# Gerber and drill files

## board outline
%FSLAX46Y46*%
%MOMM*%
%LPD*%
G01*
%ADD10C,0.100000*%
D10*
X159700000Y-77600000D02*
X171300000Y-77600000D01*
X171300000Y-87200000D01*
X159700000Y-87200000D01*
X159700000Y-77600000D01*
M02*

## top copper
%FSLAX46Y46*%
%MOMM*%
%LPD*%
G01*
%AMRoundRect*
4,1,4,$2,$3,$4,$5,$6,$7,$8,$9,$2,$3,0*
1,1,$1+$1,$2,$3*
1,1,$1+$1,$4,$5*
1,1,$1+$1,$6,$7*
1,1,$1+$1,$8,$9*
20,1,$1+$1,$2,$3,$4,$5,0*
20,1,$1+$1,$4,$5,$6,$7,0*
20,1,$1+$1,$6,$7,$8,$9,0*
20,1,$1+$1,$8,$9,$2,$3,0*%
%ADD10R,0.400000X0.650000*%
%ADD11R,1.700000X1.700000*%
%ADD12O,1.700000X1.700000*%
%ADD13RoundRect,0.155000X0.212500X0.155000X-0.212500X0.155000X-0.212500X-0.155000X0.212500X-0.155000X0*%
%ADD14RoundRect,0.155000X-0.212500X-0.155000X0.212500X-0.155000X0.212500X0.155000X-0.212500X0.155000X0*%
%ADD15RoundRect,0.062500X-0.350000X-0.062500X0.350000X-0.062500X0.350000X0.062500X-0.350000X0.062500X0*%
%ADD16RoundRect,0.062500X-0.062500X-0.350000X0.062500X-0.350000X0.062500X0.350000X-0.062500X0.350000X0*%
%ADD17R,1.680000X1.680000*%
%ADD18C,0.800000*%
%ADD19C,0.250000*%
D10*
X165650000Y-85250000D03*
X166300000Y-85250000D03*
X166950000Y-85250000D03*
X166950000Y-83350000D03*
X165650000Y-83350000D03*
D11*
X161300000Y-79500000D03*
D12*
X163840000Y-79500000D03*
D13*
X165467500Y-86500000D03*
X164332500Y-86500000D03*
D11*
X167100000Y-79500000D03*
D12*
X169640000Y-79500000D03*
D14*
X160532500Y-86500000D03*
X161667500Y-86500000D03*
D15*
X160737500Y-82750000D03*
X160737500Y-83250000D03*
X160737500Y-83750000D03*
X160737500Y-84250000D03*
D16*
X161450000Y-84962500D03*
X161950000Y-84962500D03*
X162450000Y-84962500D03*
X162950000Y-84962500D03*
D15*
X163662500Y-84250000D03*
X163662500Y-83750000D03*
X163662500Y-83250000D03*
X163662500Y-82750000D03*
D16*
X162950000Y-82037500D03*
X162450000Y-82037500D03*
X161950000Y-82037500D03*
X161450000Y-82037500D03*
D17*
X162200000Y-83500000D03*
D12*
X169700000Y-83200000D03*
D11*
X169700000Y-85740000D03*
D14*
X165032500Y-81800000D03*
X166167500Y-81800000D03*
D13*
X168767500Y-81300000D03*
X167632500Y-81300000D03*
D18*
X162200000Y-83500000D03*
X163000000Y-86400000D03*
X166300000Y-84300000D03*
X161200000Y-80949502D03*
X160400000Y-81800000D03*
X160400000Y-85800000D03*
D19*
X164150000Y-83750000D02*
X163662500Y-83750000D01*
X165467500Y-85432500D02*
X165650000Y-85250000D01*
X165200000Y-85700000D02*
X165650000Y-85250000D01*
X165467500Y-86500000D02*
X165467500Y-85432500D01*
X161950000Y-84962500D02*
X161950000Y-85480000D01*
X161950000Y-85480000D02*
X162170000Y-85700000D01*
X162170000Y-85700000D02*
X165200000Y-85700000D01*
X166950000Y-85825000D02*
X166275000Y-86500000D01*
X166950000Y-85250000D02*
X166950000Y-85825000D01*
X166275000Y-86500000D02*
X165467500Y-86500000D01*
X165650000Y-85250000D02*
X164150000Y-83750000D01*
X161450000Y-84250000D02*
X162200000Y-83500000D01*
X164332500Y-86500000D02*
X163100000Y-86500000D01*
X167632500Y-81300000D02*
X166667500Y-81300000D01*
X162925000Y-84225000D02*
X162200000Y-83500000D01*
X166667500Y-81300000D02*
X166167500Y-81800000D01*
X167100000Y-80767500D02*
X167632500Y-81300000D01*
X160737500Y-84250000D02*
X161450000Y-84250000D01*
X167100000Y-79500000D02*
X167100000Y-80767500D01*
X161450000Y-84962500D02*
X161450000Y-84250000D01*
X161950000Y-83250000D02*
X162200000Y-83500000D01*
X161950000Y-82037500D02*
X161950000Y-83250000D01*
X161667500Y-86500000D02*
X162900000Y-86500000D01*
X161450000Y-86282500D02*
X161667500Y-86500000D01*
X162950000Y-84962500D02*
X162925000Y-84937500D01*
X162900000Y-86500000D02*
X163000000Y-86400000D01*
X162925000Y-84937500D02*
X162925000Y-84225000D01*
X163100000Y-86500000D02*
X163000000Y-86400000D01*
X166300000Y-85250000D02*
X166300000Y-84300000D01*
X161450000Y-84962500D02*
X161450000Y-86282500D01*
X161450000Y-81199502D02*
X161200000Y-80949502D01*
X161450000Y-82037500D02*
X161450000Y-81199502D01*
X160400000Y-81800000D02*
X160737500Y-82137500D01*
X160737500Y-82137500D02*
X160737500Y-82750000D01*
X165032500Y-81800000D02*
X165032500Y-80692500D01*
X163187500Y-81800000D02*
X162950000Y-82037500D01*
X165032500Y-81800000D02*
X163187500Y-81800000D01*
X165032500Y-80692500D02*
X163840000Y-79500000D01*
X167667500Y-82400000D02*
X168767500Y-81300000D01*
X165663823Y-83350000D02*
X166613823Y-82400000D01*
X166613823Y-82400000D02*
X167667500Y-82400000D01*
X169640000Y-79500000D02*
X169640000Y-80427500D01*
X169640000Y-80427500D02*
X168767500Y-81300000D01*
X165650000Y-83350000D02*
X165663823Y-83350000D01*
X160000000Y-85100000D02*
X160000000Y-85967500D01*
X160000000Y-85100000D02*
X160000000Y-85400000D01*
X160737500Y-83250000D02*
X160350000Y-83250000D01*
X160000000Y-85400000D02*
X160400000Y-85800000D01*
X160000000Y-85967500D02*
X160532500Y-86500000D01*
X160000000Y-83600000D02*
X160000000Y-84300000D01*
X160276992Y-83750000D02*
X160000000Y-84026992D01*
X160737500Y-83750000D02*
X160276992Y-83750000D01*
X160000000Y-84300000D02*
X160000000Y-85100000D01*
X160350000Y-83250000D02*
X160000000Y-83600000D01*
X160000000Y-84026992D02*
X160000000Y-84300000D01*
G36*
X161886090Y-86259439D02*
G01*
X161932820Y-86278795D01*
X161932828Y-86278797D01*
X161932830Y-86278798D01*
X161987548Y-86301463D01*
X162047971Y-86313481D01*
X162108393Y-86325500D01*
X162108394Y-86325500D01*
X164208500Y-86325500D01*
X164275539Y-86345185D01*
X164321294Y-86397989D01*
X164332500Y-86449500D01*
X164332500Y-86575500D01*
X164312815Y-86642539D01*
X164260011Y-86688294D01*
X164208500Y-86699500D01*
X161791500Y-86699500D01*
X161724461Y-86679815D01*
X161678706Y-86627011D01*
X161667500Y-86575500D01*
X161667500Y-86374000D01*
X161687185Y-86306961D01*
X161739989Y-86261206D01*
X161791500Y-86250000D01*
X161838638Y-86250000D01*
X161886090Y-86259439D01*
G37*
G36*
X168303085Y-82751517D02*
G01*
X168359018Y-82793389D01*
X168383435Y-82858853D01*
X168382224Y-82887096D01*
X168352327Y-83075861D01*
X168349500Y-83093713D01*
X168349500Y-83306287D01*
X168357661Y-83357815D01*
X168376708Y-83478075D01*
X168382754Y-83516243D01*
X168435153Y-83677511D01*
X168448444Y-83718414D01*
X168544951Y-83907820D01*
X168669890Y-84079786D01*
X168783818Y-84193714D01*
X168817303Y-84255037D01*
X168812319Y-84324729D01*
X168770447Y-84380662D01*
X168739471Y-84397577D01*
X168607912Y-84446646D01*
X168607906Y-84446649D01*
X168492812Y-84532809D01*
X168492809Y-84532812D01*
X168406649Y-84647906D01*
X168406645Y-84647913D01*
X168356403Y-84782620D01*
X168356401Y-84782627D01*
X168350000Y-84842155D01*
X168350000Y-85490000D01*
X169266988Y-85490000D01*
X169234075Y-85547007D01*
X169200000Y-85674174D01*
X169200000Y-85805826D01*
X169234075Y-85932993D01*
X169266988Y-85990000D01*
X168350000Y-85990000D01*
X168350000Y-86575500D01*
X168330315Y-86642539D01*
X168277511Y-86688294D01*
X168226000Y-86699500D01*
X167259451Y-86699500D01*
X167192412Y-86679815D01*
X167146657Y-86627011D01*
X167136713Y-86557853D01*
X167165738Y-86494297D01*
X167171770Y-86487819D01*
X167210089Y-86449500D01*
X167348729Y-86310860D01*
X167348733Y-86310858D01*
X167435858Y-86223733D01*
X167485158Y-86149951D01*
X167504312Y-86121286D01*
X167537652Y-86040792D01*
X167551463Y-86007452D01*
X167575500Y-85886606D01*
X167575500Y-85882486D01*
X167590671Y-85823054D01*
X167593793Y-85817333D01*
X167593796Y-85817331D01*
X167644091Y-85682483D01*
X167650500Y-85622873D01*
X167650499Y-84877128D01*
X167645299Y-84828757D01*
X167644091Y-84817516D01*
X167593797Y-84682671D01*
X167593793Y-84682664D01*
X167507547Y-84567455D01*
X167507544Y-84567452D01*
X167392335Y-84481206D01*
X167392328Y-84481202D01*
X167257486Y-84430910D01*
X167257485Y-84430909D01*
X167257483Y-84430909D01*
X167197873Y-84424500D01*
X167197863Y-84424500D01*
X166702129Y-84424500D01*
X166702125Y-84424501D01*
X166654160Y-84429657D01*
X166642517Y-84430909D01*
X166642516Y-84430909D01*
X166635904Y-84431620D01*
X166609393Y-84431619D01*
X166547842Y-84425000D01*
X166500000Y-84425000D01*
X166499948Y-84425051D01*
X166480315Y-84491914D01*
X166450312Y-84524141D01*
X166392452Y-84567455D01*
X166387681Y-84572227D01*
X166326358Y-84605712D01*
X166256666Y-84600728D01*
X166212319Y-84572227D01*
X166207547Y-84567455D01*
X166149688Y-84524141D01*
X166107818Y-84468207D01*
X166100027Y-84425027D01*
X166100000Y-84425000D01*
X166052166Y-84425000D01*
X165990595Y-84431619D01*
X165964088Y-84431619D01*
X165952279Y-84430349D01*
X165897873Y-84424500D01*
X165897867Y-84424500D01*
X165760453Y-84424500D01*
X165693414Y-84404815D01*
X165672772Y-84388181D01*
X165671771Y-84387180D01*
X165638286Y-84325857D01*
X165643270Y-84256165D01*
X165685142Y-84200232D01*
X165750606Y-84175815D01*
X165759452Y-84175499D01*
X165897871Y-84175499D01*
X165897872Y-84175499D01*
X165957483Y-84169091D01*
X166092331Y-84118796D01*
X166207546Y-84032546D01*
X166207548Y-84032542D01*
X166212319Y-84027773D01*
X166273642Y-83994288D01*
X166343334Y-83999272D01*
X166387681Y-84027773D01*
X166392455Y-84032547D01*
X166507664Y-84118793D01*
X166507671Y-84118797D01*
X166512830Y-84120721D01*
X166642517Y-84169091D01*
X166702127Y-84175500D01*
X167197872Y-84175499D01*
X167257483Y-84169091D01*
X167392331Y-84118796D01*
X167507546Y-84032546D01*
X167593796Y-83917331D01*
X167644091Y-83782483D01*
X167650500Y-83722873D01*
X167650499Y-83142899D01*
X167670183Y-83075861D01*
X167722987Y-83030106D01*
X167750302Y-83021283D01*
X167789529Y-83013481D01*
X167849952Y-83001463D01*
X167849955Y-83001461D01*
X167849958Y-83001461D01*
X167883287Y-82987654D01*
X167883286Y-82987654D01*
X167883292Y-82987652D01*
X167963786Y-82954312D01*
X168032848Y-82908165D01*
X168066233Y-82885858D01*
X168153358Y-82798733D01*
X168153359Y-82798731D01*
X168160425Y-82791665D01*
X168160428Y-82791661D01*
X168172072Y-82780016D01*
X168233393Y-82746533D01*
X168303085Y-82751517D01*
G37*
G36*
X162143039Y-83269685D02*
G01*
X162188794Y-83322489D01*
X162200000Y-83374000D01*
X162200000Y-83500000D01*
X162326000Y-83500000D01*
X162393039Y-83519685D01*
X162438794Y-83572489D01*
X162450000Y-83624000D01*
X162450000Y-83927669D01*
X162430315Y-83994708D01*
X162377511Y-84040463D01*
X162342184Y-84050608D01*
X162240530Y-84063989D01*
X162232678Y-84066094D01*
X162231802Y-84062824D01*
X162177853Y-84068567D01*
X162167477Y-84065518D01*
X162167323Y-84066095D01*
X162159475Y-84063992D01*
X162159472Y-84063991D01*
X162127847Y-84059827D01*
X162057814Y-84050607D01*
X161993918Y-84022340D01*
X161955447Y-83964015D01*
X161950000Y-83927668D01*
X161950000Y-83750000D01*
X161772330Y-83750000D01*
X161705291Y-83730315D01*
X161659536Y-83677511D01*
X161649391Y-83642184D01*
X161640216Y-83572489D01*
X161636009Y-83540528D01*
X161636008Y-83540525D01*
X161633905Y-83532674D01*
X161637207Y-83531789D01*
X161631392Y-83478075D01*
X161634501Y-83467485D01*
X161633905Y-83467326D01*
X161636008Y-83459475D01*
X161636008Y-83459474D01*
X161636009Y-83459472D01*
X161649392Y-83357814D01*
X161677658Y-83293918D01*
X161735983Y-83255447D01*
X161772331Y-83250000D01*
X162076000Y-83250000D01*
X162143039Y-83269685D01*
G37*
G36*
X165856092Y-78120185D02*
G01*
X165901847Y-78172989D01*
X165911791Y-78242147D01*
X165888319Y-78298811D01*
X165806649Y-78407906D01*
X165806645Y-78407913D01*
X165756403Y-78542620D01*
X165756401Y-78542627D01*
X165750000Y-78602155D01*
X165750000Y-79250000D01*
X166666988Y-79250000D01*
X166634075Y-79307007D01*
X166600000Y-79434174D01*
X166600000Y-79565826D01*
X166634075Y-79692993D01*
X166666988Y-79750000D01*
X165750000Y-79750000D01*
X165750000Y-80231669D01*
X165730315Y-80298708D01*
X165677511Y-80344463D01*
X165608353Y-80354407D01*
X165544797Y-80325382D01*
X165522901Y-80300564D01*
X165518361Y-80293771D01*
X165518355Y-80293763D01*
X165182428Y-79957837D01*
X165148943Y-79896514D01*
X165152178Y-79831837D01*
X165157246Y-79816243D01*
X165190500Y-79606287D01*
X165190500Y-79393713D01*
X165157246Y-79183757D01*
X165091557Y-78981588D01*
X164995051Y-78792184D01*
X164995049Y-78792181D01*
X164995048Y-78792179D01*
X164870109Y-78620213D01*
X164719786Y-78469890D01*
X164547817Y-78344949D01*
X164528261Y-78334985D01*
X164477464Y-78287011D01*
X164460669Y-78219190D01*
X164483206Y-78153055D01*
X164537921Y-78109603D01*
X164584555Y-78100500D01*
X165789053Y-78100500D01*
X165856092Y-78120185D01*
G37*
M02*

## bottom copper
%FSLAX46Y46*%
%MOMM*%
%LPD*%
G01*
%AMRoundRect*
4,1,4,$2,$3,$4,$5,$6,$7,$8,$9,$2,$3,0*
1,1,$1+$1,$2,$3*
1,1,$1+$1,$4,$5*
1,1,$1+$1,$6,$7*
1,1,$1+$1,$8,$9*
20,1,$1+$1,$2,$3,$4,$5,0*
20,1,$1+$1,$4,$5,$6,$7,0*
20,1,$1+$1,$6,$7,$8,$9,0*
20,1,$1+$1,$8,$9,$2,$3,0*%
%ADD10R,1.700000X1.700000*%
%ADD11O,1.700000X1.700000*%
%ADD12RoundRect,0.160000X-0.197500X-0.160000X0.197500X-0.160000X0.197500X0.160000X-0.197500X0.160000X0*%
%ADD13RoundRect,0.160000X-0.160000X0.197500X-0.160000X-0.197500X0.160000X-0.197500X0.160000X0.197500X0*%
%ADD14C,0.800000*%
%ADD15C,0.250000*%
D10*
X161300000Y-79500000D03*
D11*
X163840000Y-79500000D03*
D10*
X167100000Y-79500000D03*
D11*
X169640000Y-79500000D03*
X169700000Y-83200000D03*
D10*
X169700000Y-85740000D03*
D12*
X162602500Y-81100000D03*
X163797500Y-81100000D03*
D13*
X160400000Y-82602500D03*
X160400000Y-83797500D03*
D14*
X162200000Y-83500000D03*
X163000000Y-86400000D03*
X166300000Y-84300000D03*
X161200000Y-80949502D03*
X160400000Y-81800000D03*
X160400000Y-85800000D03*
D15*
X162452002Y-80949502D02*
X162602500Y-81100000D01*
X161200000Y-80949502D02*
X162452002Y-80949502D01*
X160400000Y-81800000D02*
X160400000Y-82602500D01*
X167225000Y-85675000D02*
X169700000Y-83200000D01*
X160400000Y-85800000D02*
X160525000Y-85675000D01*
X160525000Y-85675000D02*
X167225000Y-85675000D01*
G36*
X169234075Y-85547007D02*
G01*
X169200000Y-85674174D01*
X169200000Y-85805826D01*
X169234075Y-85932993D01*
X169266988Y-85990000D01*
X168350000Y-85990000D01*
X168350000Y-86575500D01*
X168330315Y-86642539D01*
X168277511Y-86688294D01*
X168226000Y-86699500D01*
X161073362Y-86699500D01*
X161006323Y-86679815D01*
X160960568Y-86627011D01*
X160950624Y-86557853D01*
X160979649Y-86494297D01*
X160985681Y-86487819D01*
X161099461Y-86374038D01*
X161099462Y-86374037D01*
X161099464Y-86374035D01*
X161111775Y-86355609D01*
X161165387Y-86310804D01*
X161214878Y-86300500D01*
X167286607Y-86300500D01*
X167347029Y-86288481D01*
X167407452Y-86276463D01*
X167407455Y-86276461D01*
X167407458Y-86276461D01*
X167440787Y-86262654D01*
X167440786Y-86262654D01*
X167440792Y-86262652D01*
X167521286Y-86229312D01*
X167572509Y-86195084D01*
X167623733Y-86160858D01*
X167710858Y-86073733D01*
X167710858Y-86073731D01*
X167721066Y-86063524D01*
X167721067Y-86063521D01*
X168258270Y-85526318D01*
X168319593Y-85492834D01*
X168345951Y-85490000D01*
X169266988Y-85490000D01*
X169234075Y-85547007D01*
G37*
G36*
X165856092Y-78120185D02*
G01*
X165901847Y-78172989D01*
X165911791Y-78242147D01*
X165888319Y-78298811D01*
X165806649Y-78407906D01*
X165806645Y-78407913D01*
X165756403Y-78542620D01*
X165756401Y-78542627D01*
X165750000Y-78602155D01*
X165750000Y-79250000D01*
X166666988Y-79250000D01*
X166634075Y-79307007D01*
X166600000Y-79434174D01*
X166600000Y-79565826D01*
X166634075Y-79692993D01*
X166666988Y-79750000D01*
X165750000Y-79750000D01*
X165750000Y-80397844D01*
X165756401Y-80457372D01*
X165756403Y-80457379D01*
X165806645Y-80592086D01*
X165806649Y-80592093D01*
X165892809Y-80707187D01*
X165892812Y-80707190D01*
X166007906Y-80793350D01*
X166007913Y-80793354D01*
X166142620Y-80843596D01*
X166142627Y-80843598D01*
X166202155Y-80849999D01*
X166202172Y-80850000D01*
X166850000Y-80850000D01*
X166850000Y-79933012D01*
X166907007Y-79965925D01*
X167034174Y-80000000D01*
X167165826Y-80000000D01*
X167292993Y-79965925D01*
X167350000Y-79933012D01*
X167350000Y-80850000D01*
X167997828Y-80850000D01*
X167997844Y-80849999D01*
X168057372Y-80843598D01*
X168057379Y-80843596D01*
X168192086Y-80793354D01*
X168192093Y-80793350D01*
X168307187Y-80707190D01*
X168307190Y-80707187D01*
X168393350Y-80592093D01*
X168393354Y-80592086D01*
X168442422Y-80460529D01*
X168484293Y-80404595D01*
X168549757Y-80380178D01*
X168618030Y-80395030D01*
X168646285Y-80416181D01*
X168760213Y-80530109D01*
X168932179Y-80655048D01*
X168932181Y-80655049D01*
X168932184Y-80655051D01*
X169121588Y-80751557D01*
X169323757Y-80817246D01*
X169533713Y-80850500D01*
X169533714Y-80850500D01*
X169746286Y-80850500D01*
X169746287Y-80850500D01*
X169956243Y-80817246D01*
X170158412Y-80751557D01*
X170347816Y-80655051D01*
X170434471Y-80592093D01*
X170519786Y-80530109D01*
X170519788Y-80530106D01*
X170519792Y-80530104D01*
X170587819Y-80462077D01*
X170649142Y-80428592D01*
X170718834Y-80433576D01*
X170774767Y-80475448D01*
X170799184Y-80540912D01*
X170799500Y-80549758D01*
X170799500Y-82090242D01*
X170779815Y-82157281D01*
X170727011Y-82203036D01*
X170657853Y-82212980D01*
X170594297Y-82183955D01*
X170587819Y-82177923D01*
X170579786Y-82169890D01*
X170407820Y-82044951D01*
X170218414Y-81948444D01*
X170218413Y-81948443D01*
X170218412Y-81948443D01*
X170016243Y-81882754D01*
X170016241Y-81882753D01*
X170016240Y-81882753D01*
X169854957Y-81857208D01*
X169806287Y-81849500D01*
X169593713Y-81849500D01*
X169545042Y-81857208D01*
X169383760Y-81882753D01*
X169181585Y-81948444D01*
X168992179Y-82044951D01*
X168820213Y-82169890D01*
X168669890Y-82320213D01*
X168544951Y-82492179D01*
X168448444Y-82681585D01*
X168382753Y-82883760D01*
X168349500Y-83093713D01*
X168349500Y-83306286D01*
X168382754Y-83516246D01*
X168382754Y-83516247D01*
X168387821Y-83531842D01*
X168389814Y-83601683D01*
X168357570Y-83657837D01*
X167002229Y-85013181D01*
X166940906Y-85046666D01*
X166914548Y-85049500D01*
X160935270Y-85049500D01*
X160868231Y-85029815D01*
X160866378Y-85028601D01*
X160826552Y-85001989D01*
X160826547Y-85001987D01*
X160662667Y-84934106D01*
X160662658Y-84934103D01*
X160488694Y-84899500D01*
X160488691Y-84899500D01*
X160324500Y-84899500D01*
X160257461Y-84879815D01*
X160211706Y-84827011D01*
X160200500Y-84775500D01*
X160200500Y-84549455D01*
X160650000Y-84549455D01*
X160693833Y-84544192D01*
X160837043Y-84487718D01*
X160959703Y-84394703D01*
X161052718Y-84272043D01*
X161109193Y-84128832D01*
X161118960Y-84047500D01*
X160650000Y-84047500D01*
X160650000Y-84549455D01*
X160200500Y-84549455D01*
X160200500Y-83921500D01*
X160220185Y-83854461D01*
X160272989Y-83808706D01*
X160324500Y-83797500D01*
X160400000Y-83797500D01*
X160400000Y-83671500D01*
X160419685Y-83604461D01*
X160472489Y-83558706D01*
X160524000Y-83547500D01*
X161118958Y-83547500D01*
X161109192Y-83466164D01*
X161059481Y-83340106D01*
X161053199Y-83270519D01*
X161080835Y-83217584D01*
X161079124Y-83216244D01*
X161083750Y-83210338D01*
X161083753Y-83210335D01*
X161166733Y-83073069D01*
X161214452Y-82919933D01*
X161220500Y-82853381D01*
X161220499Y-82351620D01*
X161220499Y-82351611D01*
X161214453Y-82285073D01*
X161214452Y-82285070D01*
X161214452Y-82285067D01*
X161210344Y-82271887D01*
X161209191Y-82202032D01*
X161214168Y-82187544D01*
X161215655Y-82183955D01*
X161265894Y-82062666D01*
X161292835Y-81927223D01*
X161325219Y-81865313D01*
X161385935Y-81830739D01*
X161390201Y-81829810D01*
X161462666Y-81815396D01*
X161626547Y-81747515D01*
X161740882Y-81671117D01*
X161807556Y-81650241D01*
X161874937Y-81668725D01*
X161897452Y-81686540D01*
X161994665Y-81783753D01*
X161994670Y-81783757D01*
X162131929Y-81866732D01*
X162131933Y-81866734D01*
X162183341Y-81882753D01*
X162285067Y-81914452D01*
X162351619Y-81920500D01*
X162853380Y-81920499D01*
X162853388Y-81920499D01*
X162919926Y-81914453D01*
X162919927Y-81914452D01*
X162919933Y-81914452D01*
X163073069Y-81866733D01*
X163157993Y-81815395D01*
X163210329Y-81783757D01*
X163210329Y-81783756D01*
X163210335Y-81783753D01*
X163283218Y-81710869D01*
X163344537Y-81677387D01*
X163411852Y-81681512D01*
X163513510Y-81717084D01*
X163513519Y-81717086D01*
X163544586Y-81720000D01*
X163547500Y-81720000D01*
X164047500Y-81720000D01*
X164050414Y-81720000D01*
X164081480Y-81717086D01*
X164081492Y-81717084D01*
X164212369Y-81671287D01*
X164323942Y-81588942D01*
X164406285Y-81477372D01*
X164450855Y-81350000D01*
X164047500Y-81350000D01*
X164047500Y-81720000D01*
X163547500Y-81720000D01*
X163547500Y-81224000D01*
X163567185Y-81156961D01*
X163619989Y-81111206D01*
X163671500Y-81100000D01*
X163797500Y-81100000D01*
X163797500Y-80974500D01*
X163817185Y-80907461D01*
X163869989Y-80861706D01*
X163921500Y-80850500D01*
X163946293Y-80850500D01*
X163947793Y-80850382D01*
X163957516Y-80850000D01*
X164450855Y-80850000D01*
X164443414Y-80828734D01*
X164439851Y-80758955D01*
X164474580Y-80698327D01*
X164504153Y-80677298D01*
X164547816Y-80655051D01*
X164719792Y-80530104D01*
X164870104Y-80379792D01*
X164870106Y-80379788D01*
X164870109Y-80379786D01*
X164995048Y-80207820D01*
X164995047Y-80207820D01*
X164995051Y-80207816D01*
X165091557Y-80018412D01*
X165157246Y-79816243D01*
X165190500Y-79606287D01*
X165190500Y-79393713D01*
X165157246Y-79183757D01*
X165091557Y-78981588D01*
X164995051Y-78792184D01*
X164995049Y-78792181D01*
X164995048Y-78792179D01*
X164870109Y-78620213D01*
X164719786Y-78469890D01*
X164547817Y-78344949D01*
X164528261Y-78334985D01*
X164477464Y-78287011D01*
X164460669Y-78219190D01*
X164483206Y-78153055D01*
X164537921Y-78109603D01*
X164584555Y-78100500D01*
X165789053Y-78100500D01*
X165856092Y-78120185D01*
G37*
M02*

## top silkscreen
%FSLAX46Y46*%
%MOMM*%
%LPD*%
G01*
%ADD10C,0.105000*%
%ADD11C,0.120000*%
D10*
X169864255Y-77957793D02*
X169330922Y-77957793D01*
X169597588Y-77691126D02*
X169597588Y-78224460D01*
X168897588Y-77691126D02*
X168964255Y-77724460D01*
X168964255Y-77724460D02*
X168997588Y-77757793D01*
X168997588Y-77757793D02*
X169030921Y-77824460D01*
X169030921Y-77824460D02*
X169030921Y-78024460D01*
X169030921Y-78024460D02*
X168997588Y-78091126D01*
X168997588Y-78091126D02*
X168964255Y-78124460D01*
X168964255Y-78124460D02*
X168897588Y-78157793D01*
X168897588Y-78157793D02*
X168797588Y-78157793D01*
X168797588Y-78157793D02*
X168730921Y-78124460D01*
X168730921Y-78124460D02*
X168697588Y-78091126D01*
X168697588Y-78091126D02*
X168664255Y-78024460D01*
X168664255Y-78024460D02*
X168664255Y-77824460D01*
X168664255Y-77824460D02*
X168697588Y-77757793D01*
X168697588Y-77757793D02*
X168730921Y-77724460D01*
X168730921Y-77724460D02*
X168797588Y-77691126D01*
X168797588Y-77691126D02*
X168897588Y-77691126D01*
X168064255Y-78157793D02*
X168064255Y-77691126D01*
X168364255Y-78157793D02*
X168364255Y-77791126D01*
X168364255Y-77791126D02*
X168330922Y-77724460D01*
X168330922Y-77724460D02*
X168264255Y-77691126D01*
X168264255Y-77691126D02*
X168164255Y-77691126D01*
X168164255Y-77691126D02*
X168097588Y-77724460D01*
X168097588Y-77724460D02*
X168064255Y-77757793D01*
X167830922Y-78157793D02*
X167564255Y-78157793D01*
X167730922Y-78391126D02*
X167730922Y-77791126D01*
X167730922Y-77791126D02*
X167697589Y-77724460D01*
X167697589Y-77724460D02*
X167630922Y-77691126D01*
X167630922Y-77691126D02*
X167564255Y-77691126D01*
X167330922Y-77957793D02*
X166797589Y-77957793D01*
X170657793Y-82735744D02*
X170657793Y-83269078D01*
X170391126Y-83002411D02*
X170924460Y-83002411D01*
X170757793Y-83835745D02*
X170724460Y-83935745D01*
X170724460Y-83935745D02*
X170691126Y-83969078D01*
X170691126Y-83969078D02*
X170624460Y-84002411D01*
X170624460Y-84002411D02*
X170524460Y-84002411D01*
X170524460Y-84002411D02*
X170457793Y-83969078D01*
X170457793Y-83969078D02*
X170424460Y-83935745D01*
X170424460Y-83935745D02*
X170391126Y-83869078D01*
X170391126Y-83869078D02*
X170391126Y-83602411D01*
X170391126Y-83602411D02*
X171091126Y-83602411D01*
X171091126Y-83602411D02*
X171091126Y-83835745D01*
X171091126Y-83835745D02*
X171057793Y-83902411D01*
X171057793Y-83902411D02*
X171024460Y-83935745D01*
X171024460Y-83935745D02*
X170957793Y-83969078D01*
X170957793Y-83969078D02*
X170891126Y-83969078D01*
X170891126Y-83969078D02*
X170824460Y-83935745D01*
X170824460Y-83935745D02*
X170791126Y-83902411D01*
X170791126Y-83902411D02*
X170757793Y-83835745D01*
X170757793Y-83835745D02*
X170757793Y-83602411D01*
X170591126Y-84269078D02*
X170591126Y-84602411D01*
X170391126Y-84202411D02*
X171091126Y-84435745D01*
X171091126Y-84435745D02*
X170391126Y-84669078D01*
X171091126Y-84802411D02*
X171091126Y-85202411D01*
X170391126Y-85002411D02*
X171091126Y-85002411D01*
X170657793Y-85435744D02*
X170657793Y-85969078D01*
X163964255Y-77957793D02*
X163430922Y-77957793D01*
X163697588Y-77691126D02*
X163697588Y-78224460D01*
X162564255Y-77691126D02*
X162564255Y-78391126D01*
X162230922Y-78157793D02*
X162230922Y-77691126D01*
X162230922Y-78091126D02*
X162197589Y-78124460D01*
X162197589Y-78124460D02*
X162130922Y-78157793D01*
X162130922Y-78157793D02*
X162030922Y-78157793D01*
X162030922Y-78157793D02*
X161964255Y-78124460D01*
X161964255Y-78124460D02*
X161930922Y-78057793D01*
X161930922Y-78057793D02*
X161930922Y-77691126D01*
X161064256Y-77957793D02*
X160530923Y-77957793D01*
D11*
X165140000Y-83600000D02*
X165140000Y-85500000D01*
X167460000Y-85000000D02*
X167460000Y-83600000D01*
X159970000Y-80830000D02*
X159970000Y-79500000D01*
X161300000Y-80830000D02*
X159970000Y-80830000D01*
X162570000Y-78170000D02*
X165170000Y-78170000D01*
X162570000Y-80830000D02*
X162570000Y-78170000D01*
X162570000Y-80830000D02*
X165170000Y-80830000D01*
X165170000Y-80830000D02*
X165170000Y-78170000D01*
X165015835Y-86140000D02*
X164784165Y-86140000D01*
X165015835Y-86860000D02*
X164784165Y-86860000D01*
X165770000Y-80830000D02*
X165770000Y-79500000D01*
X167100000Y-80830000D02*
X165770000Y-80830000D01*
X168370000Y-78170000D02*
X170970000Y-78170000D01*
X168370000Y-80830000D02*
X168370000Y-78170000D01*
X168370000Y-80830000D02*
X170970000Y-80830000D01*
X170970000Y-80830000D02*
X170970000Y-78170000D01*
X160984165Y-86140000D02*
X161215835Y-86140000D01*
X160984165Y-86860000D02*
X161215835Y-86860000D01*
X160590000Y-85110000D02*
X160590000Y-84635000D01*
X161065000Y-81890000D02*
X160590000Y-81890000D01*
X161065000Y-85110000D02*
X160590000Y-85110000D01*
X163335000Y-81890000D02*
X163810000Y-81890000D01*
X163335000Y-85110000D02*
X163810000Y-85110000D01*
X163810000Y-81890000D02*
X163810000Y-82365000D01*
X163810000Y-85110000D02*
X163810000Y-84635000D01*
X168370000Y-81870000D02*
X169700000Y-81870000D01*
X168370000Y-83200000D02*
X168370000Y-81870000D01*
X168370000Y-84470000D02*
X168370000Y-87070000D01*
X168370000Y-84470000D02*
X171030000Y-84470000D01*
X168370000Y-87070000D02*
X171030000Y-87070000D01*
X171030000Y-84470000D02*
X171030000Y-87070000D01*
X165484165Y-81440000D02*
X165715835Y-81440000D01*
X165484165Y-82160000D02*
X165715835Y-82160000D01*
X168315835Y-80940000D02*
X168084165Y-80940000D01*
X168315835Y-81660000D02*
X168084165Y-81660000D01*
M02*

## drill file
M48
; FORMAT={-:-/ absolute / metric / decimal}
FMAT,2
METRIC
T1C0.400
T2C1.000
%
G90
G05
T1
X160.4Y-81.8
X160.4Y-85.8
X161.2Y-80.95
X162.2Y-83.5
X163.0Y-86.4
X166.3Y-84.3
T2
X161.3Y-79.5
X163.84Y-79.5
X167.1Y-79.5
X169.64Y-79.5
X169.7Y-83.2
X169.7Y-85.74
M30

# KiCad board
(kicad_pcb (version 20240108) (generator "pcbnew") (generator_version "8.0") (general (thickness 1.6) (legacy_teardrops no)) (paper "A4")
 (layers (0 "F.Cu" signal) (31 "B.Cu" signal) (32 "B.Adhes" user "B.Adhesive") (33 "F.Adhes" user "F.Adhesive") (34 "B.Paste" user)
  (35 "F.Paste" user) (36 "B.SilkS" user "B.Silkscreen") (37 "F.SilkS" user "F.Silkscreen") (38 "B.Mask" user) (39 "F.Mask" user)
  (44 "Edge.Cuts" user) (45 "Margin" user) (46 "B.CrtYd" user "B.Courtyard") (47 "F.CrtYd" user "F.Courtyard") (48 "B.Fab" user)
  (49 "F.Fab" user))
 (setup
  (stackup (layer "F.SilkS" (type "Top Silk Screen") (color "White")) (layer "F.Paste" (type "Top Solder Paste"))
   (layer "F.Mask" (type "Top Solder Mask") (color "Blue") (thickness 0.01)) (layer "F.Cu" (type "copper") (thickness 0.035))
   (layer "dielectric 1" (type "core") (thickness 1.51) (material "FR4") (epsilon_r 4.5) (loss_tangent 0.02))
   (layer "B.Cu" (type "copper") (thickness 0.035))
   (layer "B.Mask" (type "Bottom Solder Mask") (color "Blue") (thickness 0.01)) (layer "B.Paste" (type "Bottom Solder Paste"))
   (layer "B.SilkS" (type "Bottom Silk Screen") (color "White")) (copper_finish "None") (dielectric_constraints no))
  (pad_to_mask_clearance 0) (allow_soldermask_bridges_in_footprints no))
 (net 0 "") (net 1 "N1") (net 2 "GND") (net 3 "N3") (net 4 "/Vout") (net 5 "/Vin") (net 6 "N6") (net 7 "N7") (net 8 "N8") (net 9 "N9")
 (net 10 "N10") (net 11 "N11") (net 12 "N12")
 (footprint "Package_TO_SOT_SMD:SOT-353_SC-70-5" (layer "F.Cu") (at 166.3 84.3 90)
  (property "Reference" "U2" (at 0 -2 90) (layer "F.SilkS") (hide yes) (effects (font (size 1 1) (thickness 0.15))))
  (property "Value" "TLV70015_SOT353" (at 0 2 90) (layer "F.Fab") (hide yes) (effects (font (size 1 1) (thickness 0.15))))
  (fp_line (start 0.7 -1.16) (end -1.2 -1.16) (stroke (width 0.12) (type solid)) (layer "F.SilkS"))
  (fp_line (start -0.7 1.16) (end 0.7 1.16) (stroke (width 0.12) (type solid)) (layer "F.SilkS"))
  (pad "1" smd rect (at -0.95 -0.65 90) (size 0.65 0.4) (layers "F.Cu" "F.Paste" "F.Mask") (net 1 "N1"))
  (pad "2" smd rect (at -0.95 0 90) (size 0.65 0.4) (layers "F.Cu" "F.Paste" "F.Mask") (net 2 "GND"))
  (pad "3" smd rect (at -0.95 0.65 90) (size 0.65 0.4) (layers "F.Cu" "F.Paste" "F.Mask") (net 1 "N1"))
  (pad "4" smd rect (at 0.95 0.65 90) (size 0.65 0.4) (layers "F.Cu" "F.Paste" "F.Mask") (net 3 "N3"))
  (pad "5" smd rect (at 0.95 -0.65 90) (size 0.65 0.4) (layers "F.Cu" "F.Paste" "F.Mask") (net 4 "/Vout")))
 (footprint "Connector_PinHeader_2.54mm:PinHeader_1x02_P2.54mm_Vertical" (layer "F.Cu") (at 161.3 79.5 90)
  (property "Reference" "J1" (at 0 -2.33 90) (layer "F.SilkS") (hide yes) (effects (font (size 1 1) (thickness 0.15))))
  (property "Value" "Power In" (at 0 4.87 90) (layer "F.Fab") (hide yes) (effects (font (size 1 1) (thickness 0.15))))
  (fp_line (start -1.33 -1.33) (end 0 -1.33) (stroke (width 0.12) (type solid)) (layer "F.SilkS"))
  (fp_line (start -1.33 0) (end -1.33 -1.33) (stroke (width 0.12) (type solid)) (layer "F.SilkS"))
  (fp_line (start 1.33 1.27) (end 1.33 3.87) (stroke (width 0.12) (type solid)) (layer "F.SilkS"))
  (fp_line (start -1.33 1.27) (end 1.33 1.27) (stroke (width 0.12) (type solid)) (layer "F.SilkS"))
  (fp_line (start -1.33 1.27) (end -1.33 3.87) (stroke (width 0.12) (type solid)) (layer "F.SilkS"))
  (fp_line (start -1.33 3.87) (end 1.33 3.87) (stroke (width 0.12) (type solid)) (layer "F.SilkS"))
  (pad "1" thru_hole rect (at 0 0 90) (size 1.7 1.7) (drill 1) (layers "*.Cu" "*.Mask") (remove_unused_layers no) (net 2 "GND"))
  (pad "2" thru_hole oval (at 0 2.54 90) (size 1.7 1.7) (drill 1) (layers "*.Cu" "*.Mask") (remove_unused_layers no) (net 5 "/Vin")))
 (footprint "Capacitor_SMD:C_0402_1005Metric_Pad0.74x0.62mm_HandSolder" (layer "F.Cu") (at 164.9 86.5 180)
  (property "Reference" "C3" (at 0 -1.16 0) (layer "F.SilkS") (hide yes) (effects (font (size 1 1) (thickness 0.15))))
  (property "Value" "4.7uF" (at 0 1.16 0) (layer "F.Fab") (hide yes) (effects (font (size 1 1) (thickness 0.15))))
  (fp_line (start -0.115835 0.36) (end 0.115835 0.36) (stroke (width 0.12) (type solid)) (layer "F.SilkS"))
  (fp_line (start -0.115835 -0.36) (end 0.115835 -0.36) (stroke (width 0.12) (type solid)) (layer "F.SilkS"))
  (pad "1" smd roundrect (at -0.5675 0 180) (size 0.735 0.62) (layers "F.Cu" "F.Paste" "F.Mask") (roundrect_rratio 0.25) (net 1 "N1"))
  (pad "2" smd roundrect (at 0.5675 0 180) (size 0.735 0.62) (layers "F.Cu" "F.Paste" "F.Mask") (roundrect_rratio 0.25) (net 2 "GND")))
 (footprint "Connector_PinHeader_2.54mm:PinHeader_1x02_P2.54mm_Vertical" (layer "F.Cu") (at 167.1 79.5 90)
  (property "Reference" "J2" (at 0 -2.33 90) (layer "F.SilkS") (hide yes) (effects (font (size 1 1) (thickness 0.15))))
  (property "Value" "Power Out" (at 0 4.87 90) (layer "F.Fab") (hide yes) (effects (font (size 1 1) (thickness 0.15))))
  (fp_line (start -1.33 -1.33) (end 0 -1.33) (stroke (width 0.12) (type solid)) (layer "F.SilkS"))
  (fp_line (start -1.33 0) (end -1.33 -1.33) (stroke (width 0.12) (type solid)) (layer "F.SilkS"))
  (fp_line (start 1.33 1.27) (end 1.33 3.87) (stroke (width 0.12) (type solid)) (layer "F.SilkS"))
  (fp_line (start -1.33 1.27) (end 1.33 1.27) (stroke (width 0.12) (type solid)) (layer "F.SilkS"))
  (fp_line (start -1.33 1.27) (end -1.33 3.87) (stroke (width 0.12) (type solid)) (layer "F.SilkS"))
  (fp_line (start -1.33 3.87) (end 1.33 3.87) (stroke (width 0.12) (type solid)) (layer "F.SilkS"))
  (pad "1" thru_hole rect (at 0 0 90) (size 1.7 1.7) (drill 1) (layers "*.Cu" "*.Mask") (remove_unused_layers no) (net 2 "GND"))
  (pad "2" thru_hole oval (at 0 2.54 90) (size 1.7 1.7) (drill 1) (layers "*.Cu" "*.Mask") (remove_unused_layers no) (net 4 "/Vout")))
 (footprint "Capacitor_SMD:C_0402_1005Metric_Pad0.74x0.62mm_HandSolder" (layer "F.Cu") (at 161.1 86.5)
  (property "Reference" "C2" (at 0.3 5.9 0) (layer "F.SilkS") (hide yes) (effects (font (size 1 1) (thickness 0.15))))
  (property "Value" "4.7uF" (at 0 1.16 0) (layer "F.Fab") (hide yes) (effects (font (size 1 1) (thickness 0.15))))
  (fp_line (start -0.115835 -0.36) (end 0.115835 -0.36) (stroke (width 0.12) (type solid)) (layer "F.SilkS"))
  (fp_line (start -0.115835 0.36) (end 0.115835 0.36) (stroke (width 0.12) (type solid)) (layer "F.SilkS"))
  (pad "1" smd roundrect (at -0.5675 0) (size 0.735 0.62) (layers "F.Cu" "F.Paste" "F.Mask") (roundrect_rratio 0.25) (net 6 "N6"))
  (pad "2" smd roundrect (at 0.5675 0) (size 0.735 0.62) (layers "F.Cu" "F.Paste" "F.Mask") (roundrect_rratio 0.25) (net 2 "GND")))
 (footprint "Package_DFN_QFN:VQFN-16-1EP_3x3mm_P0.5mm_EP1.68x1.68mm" (layer "F.Cu") (at 162.2 83.5)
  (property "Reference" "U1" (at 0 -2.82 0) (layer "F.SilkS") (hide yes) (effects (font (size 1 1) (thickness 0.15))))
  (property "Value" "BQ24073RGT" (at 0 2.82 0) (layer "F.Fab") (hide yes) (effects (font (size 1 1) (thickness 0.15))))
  (fp_line (start -1.61 1.61) (end -1.61 1.135) (stroke (width 0.12) (type solid)) (layer "F.SilkS"))
  (fp_line (start -1.135 -1.61) (end -1.61 -1.61) (stroke (width 0.12) (type solid)) (layer "F.SilkS"))
  (fp_line (start -1.135 1.61) (end -1.61 1.61) (stroke (width 0.12) (type solid)) (layer "F.SilkS"))
  (fp_line (start 1.135 -1.61) (end 1.61 -1.61) (stroke (width 0.12) (type solid)) (layer "F.SilkS"))
  (fp_line (start 1.135 1.61) (end 1.61 1.61) (stroke (width 0.12) (type solid)) (layer "F.SilkS"))
  (fp_line (start 1.61 -1.61) (end 1.61 -1.135) (stroke (width 0.12) (type solid)) (layer "F.SilkS"))
  (fp_line (start 1.61 1.61) (end 1.61 1.135) (stroke (width 0.12) (type solid)) (layer "F.SilkS"))
  (pad "" smd roundrect (at -0.42 -0.42) (size 0.68 0.68) (layers "F.Paste") (roundrect_rratio 0.25))
  (pad "" smd roundrect (at -0.42 0.42) (size 0.68 0.68) (layers "F.Paste") (roundrect_rratio 0.25))
  (pad "" smd roundrect (at 0.42 -0.42) (size 0.68 0.68) (layers "F.Paste") (roundrect_rratio 0.25))
  (pad "" smd roundrect (at 0.42 0.42) (size 0.68 0.68) (layers "F.Paste") (roundrect_rratio 0.25))
  (pad "1" smd roundrect (at -1.4625 -0.75) (size 0.825 0.25) (layers "F.Cu" "F.Paste" "F.Mask") (roundrect_rratio 0.25) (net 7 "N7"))
  (pad "2" smd roundrect (at -1.4625 -0.25) (size 0.825 0.25) (layers "F.Cu" "F.Paste" "F.Mask") (roundrect_rratio 0.25) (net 6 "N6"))
  (pad "3" smd roundrect (at -1.4625 0.25) (size 0.825 0.25) (layers "F.Cu" "F.Paste" "F.Mask") (roundrect_rratio 0.25) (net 6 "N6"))
  (pad "4" smd roundrect (at -1.4625 0.75) (size 0.825 0.25) (layers "F.Cu" "F.Paste" "F.Mask") (roundrect_rratio 0.25) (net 2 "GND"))
  (pad "5" smd roundrect (at -0.75 1.4625) (size 0.25 0.825) (layers "F.Cu" "F.Paste" "F.Mask") (roundrect_rratio 0.25) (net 2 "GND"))
  (pad "6" smd roundrect (at -0.25 1.4625) (size 0.25 0.825) (layers "F.Cu" "F.Paste" "F.Mask") (roundrect_rratio 0.25) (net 1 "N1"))
  (pad "7" smd roundrect (at 0.25 1.4625) (size 0.25 0.825) (layers "F.Cu" "F.Paste" "F.Mask") (roundrect_rratio 0.25) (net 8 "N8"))
  (pad "8" smd roundrect (at 0.75 1.4625) (size 0.25 0.825) (layers "F.Cu" "F.Paste" "F.Mask") (roundrect_rratio 0.25) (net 2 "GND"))
  (pad "9" smd roundrect (at 1.4625 0.75) (size 0.825 0.25) (layers "F.Cu" "F.Paste" "F.Mask") (roundrect_rratio 0.25) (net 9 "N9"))
  (pad "10" smd roundrect (at 1.4625 0.25) (size 0.825 0.25) (layers "F.Cu" "F.Paste" "F.Mask") (roundrect_rratio 0.25) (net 1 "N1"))
  (pad "11" smd roundrect (at 1.4625 -0.25) (size 0.825 0.25) (layers "F.Cu" "F.Paste" "F.Mask") (roundrect_rratio 0.25) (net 1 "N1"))
  (pad "12" smd roundrect (at 1.4625 -0.75) (size 0.825 0.25) (layers "F.Cu" "F.Paste" "F.Mask") (roundrect_rratio 0.25) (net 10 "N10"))
  (pad "13" smd roundrect (at 0.75 -1.4625) (size 0.25 0.825) (layers "F.Cu" "F.Paste" "F.Mask") (roundrect_rratio 0.25) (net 5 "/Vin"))
  (pad "14" smd roundrect (at 0.25 -1.4625) (size 0.25 0.825) (layers "F.Cu" "F.Paste" "F.Mask") (roundrect_rratio 0.25) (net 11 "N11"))
  (pad "15" smd roundrect (at -0.25 -1.4625) (size 0.25 0.825) (layers "F.Cu" "F.Paste" "F.Mask") (roundrect_rratio 0.25) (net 2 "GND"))
  (pad "16" smd roundrect (at -0.75 -1.4625) (size 0.25 0.825) (layers "F.Cu" "F.Paste" "F.Mask") (roundrect_rratio 0.25) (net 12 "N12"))
  (pad "17" smd rect (at 0 0) (size 1.68 1.68) (layers "F.Cu" "F.Mask") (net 2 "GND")))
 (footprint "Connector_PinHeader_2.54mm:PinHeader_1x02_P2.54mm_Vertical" (layer "F.Cu") (at 169.7 83.2)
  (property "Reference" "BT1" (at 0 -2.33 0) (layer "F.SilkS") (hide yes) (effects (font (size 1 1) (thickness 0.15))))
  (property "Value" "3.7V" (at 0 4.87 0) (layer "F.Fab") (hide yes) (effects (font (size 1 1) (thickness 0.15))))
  (fp_line (start -1.33 -1.33) (end 0 -1.33) (stroke (width 0.12) (type solid)) (layer "F.SilkS"))
  (fp_line (start -1.33 0) (end -1.33 -1.33) (stroke (width 0.12) (type solid)) (layer "F.SilkS"))
  (fp_line (start -1.33 1.27) (end -1.33 3.87) (stroke (width 0.12) (type solid)) (layer "F.SilkS"))
  (fp_line (start -1.33 1.27) (end 1.33 1.27) (stroke (width 0.12) (type solid)) (layer "F.SilkS"))
  (fp_line (start -1.33 3.87) (end 1.33 3.87) (stroke (width 0.12) (type solid)) (layer "F.SilkS"))
  (fp_line (start 1.33 1.27) (end 1.33 3.87) (stroke (width 0.12) (type solid)) (layer "F.SilkS"))
  (pad "1" thru_hole oval (at 0 0) (size 1.7 1.7) (drill 1) (layers "*.Cu" "*.Mask") (remove_unused_layers no) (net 6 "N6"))
  (pad "2" thru_hole rect (at 0 2.54) (size 1.7 1.7) (drill 1) (layers "*.Cu" "*.Mask") (remove_unused_layers no) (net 2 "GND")))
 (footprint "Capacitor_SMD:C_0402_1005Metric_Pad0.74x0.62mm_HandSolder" (layer "F.Cu") (at 165.6 81.8)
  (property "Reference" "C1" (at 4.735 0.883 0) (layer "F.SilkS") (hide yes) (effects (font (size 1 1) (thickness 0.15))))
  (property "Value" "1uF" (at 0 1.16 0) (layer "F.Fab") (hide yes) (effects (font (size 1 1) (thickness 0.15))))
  (fp_line (start -0.115835 -0.36) (end 0.115835 -0.36) (stroke (width 0.12) (type solid)) (layer "F.SilkS"))
  (fp_line (start -0.115835 0.36) (end 0.115835 0.36) (stroke (width 0.12) (type solid)) (layer "F.SilkS"))
  (pad "1" smd roundrect (at -0.5675 0) (size 0.735 0.62) (layers "F.Cu" "F.Paste" "F.Mask") (roundrect_rratio 0.25) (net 5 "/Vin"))
  (pad "2" smd roundrect (at 0.5675 0) (size 0.735 0.62) (layers "F.Cu" "F.Paste" "F.Mask") (roundrect_rratio 0.25) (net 2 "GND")))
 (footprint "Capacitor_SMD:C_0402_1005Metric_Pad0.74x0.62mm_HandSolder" (layer "F.Cu") (at 168.2 81.3 180)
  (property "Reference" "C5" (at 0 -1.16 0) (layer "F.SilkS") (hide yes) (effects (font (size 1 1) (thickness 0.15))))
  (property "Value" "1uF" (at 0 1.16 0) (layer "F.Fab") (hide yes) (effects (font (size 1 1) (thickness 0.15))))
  (fp_line (start -0.115835 0.36) (end 0.115835 0.36) (stroke (width 0.12) (type solid)) (layer "F.SilkS"))
  (fp_line (start -0.115835 -0.36) (end 0.115835 -0.36) (stroke (width 0.12) (type solid)) (layer "F.SilkS"))
  (pad "1" smd roundrect (at -0.5675 0 180) (size 0.735 0.62) (layers "F.Cu" "F.Paste" "F.Mask") (roundrect_rratio 0.25) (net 4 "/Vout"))
  (pad "2" smd roundrect (at 0.5675 0 180) (size 0.735 0.62) (layers "F.Cu" "F.Paste" "F.Mask") (roundrect_rratio 0.25) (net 2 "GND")))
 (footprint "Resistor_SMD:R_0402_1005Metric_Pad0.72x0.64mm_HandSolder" (layer "B.Cu") (at 163.2 81.1)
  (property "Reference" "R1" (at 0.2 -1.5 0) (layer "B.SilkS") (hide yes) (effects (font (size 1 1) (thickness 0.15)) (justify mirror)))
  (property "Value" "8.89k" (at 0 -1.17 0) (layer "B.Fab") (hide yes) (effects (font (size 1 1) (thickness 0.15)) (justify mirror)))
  (pad "1" smd roundrect (at -0.5975 0) (size 0.715 0.64) (layers "B.Cu" "B.Paste" "B.Mask") (roundrect_rratio 0.25) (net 12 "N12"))
  (pad "2" smd roundrect (at 0.5975 0) (size 0.715 0.64) (layers "B.Cu" "B.Paste" "B.Mask") (roundrect_rratio 0.25) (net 2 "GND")
   (zone_connect 1) (thermal_bridge_width 0.5) (thermal_gap 0.3)))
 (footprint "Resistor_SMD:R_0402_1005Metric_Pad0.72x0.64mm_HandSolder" (layer "B.Cu") (at 160.4 83.2 -90)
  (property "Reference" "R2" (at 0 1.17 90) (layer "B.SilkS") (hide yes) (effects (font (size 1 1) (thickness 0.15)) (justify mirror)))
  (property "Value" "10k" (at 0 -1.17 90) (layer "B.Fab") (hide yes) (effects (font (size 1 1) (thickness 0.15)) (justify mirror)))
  (pad "1" smd roundrect (at -0.5975 0 270) (size 0.715 0.64) (layers "B.Cu" "B.Paste" "B.Mask") (roundrect_rratio 0.25) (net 7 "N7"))
  (pad "2" smd roundrect (at 0.5975 0 270) (size 0.715 0.64) (layers "B.Cu" "B.Paste" "B.Mask") (roundrect_rratio 0.25) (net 2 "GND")
   (zone_connect 1) (thermal_bridge_width 0.5) (thermal_gap 0.4)))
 (gr_rect (start 159.7 77.6) (end 171.3 87.2) (stroke (width 0.1) (type default)) (fill none) (layer "Edge.Cuts"))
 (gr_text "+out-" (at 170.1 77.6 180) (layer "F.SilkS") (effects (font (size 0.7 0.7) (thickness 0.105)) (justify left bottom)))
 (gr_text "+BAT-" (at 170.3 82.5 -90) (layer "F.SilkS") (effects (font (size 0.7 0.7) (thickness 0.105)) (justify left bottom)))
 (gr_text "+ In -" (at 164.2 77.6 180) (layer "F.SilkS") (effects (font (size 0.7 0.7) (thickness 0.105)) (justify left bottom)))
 (segment (start 164.15 83.75) (end 163.6625 83.75) (width 0.25) (layer "F.Cu") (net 1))
 (segment (start 165.4675 85.4325) (end 165.65 85.25) (width 0.25) (layer "F.Cu") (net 1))
 (segment (start 165.2 85.7) (end 165.65 85.25) (width 0.25) (layer "F.Cu") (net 1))
 (segment (start 165.4675 86.5) (end 165.4675 85.4325) (width 0.25) (layer "F.Cu") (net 1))
 (segment (start 161.95 84.9625) (end 161.95 85.48) (width 0.25) (layer "F.Cu") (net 1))
 (segment (start 161.95 85.48) (end 162.17 85.7) (width 0.25) (layer "F.Cu") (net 1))
 (segment (start 162.17 85.7) (end 165.2 85.7) (width 0.25) (layer "F.Cu") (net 1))
 (segment (start 166.95 85.825) (end 166.275 86.5) (width 0.25) (layer "F.Cu") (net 1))
 (segment (start 166.95 85.25) (end 166.95 85.825) (width 0.25) (layer "F.Cu") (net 1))
 (segment (start 166.275 86.5) (end 165.4675 86.5) (width 0.25) (layer "F.Cu") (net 1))
 (segment (start 165.65 85.25) (end 164.15 83.75) (width 0.25) (layer "F.Cu") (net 1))
 (segment (start 161.45 84.25) (end 162.2 83.5) (width 0.25) (layer "F.Cu") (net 2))
 (segment (start 164.3325 86.5) (end 163.1 86.5) (width 0.25) (layer "F.Cu") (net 2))
 (segment (start 167.6325 81.3) (end 166.6675 81.3) (width 0.25) (layer "F.Cu") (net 2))
 (segment (start 162.925 84.225) (end 162.2 83.5) (width 0.25) (layer "F.Cu") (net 2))
 (segment (start 166.6675 81.3) (end 166.1675 81.8) (width 0.25) (layer "F.Cu") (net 2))
 (segment (start 167.1 80.7675) (end 167.6325 81.3) (width 0.25) (layer "F.Cu") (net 2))
 (segment (start 160.7375 84.25) (end 161.45 84.25) (width 0.25) (layer "F.Cu") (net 2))
 (segment (start 167.1 79.5) (end 167.1 80.7675) (width 0.25) (layer "F.Cu") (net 2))
 (segment (start 161.45 84.9625) (end 161.45 84.25) (width 0.25) (layer "F.Cu") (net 2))
 (segment (start 161.95 83.25) (end 162.2 83.5) (width 0.25) (layer "F.Cu") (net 2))
 (segment (start 161.95 82.0375) (end 161.95 83.25) (width 0.25) (layer "F.Cu") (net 2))
 (segment (start 161.6675 86.5) (end 162.9 86.5) (width 0.25) (layer "F.Cu") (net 2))
 (segment (start 161.45 86.2825) (end 161.6675 86.5) (width 0.25) (layer "F.Cu") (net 2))
 (segment (start 162.95 84.9625) (end 162.925 84.9375) (width 0.25) (layer "F.Cu") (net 2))
 (segment (start 162.9 86.5) (end 163 86.4) (width 0.25) (layer "F.Cu") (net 2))
 (segment (start 162.925 84.9375) (end 162.925 84.225) (width 0.25) (layer "F.Cu") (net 2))
 (segment (start 163.1 86.5) (end 163 86.4) (width 0.25) (layer "F.Cu") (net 2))
 (segment (start 166.3 85.25) (end 166.3 84.3) (width 0.25) (layer "F.Cu") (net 2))
 (segment (start 161.45 84.9625) (end 161.45 86.2825) (width 0.25) (layer "F.Cu") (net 2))
 (via (at 162.2 83.5) (size 0.8) (drill 0.4) (layers "F.Cu" "B.Cu") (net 2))
 (via (at 163 86.4) (size 0.8) (drill 0.4) (layers "F.Cu" "B.Cu") (free yes) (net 2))
 (via (at 166.3 84.3) (size 0.8) (drill 0.4) (layers "F.Cu" "B.Cu") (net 2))
 (segment (start 161.45 81.199502) (end 161.2 80.949502) (width 0.25) (layer "F.Cu") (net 12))
 (segment (start 161.45 82.0375) (end 161.45 81.199502) (width 0.25) (layer "F.Cu") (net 12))
 (via (at 161.2 80.949502) (size 0.8) (drill 0.4) (layers "F.Cu" "B.Cu") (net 12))
 (segment (start 162.452002 80.949502) (end 162.6025 81.1) (width 0.25) (layer "B.Cu") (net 12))
 (segment (start 161.2 80.949502) (end 162.452002 80.949502) (width 0.25) (layer "B.Cu") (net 12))
 (segment (start 160.4 81.8) (end 160.7375 82.1375) (width 0.25) (layer "F.Cu") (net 7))
 (segment (start 160.7375 82.1375) (end 160.7375 82.75) (width 0.25) (layer "F.Cu") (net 7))
 (via (at 160.4 81.8) (size 0.8) (drill 0.4) (layers "F.Cu" "B.Cu") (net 7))
 (segment (start 160.4 81.8) (end 160.4 82.6025) (width 0.25) (layer "B.Cu") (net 7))
 (segment (start 165.0325 81.8) (end 165.0325 80.6925) (width 0.25) (layer "F.Cu") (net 5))
 (segment (start 163.1875 81.8) (end 162.95 82.0375) (width 0.25) (layer "F.Cu") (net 5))
 (segment (start 165.0325 81.8) (end 163.1875 81.8) (width 0.25) (layer "F.Cu") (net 5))
 (segment (start 165.0325 80.6925) (end 163.84 79.5) (width 0.25) (layer "F.Cu") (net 5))
 (segment (start 167.6675 82.4) (end 168.7675 81.3) (width 0.25) (layer "F.Cu") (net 4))
 (segment (start 165.663823 83.35) (end 166.613823 82.4) (width 0.25) (layer "F.Cu") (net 4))
 (segment (start 166.613823 82.4) (end 167.6675 82.4) (width 0.25) (layer "F.Cu") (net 4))
 (segment (start 169.64 79.5) (end 169.64 80.4275) (width 0.25) (layer "F.Cu") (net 4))
 (segment (start 169.64 80.4275) (end 168.7675 81.3) (width 0.25) (layer "F.Cu") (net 4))
 (segment (start 165.65 83.35) (end 165.663823 83.35) (width 0.25) (layer "F.Cu") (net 4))
 (segment (start 160 85.1) (end 160 85.9675) (width 0.25) (layer "F.Cu") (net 6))
 (segment (start 160 85.1) (end 160 85.4) (width 0.25) (layer "F.Cu") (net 6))
 (segment (start 160.7375 83.25) (end 160.35 83.25) (width 0.25) (layer "F.Cu") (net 6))
 (segment (start 160 85.4) (end 160.4 85.8) (width 0.25) (layer "F.Cu") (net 6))
 (segment (start 160 85.9675) (end 160.5325 86.5) (width 0.25) (layer "F.Cu") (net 6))
 (segment (start 160 83.6) (end 160 84.3) (width 0.25) (layer "F.Cu") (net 6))
 (segment (start 160.276992 83.75) (end 160 84.026992) (width 0.25) (layer "F.Cu") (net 6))
 (segment (start 160.7375 83.75) (end 160.276992 83.75) (width 0.25) (layer "F.Cu") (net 6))
 (segment (start 160 84.3) (end 160 85.1) (width 0.25) (layer "F.Cu") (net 6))
 (segment (start 160.35 83.25) (end 160 83.6) (width 0.25) (layer "F.Cu") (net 6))
 (segment (start 160 84.026992) (end 160 84.3) (width 0.25) (layer "F.Cu") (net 6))
 (via (at 160.4 85.8) (size 0.8) (drill 0.4) (layers "F.Cu" "B.Cu") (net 6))
 (segment (start 167.225 85.675) (end 169.7 83.2) (width 0.25) (layer "B.Cu") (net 6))
 (segment (start 160.4 85.8) (end 160.525 85.675) (width 0.25) (layer "B.Cu") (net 6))
 (segment (start 160.525 85.675) (end 167.225 85.675) (width 0.25) (layer "B.Cu") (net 6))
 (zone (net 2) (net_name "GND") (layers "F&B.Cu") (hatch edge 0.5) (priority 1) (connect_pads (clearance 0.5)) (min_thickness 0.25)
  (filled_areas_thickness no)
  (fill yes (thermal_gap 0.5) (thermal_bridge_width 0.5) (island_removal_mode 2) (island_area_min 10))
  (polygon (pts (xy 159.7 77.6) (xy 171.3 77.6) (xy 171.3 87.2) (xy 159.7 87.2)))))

